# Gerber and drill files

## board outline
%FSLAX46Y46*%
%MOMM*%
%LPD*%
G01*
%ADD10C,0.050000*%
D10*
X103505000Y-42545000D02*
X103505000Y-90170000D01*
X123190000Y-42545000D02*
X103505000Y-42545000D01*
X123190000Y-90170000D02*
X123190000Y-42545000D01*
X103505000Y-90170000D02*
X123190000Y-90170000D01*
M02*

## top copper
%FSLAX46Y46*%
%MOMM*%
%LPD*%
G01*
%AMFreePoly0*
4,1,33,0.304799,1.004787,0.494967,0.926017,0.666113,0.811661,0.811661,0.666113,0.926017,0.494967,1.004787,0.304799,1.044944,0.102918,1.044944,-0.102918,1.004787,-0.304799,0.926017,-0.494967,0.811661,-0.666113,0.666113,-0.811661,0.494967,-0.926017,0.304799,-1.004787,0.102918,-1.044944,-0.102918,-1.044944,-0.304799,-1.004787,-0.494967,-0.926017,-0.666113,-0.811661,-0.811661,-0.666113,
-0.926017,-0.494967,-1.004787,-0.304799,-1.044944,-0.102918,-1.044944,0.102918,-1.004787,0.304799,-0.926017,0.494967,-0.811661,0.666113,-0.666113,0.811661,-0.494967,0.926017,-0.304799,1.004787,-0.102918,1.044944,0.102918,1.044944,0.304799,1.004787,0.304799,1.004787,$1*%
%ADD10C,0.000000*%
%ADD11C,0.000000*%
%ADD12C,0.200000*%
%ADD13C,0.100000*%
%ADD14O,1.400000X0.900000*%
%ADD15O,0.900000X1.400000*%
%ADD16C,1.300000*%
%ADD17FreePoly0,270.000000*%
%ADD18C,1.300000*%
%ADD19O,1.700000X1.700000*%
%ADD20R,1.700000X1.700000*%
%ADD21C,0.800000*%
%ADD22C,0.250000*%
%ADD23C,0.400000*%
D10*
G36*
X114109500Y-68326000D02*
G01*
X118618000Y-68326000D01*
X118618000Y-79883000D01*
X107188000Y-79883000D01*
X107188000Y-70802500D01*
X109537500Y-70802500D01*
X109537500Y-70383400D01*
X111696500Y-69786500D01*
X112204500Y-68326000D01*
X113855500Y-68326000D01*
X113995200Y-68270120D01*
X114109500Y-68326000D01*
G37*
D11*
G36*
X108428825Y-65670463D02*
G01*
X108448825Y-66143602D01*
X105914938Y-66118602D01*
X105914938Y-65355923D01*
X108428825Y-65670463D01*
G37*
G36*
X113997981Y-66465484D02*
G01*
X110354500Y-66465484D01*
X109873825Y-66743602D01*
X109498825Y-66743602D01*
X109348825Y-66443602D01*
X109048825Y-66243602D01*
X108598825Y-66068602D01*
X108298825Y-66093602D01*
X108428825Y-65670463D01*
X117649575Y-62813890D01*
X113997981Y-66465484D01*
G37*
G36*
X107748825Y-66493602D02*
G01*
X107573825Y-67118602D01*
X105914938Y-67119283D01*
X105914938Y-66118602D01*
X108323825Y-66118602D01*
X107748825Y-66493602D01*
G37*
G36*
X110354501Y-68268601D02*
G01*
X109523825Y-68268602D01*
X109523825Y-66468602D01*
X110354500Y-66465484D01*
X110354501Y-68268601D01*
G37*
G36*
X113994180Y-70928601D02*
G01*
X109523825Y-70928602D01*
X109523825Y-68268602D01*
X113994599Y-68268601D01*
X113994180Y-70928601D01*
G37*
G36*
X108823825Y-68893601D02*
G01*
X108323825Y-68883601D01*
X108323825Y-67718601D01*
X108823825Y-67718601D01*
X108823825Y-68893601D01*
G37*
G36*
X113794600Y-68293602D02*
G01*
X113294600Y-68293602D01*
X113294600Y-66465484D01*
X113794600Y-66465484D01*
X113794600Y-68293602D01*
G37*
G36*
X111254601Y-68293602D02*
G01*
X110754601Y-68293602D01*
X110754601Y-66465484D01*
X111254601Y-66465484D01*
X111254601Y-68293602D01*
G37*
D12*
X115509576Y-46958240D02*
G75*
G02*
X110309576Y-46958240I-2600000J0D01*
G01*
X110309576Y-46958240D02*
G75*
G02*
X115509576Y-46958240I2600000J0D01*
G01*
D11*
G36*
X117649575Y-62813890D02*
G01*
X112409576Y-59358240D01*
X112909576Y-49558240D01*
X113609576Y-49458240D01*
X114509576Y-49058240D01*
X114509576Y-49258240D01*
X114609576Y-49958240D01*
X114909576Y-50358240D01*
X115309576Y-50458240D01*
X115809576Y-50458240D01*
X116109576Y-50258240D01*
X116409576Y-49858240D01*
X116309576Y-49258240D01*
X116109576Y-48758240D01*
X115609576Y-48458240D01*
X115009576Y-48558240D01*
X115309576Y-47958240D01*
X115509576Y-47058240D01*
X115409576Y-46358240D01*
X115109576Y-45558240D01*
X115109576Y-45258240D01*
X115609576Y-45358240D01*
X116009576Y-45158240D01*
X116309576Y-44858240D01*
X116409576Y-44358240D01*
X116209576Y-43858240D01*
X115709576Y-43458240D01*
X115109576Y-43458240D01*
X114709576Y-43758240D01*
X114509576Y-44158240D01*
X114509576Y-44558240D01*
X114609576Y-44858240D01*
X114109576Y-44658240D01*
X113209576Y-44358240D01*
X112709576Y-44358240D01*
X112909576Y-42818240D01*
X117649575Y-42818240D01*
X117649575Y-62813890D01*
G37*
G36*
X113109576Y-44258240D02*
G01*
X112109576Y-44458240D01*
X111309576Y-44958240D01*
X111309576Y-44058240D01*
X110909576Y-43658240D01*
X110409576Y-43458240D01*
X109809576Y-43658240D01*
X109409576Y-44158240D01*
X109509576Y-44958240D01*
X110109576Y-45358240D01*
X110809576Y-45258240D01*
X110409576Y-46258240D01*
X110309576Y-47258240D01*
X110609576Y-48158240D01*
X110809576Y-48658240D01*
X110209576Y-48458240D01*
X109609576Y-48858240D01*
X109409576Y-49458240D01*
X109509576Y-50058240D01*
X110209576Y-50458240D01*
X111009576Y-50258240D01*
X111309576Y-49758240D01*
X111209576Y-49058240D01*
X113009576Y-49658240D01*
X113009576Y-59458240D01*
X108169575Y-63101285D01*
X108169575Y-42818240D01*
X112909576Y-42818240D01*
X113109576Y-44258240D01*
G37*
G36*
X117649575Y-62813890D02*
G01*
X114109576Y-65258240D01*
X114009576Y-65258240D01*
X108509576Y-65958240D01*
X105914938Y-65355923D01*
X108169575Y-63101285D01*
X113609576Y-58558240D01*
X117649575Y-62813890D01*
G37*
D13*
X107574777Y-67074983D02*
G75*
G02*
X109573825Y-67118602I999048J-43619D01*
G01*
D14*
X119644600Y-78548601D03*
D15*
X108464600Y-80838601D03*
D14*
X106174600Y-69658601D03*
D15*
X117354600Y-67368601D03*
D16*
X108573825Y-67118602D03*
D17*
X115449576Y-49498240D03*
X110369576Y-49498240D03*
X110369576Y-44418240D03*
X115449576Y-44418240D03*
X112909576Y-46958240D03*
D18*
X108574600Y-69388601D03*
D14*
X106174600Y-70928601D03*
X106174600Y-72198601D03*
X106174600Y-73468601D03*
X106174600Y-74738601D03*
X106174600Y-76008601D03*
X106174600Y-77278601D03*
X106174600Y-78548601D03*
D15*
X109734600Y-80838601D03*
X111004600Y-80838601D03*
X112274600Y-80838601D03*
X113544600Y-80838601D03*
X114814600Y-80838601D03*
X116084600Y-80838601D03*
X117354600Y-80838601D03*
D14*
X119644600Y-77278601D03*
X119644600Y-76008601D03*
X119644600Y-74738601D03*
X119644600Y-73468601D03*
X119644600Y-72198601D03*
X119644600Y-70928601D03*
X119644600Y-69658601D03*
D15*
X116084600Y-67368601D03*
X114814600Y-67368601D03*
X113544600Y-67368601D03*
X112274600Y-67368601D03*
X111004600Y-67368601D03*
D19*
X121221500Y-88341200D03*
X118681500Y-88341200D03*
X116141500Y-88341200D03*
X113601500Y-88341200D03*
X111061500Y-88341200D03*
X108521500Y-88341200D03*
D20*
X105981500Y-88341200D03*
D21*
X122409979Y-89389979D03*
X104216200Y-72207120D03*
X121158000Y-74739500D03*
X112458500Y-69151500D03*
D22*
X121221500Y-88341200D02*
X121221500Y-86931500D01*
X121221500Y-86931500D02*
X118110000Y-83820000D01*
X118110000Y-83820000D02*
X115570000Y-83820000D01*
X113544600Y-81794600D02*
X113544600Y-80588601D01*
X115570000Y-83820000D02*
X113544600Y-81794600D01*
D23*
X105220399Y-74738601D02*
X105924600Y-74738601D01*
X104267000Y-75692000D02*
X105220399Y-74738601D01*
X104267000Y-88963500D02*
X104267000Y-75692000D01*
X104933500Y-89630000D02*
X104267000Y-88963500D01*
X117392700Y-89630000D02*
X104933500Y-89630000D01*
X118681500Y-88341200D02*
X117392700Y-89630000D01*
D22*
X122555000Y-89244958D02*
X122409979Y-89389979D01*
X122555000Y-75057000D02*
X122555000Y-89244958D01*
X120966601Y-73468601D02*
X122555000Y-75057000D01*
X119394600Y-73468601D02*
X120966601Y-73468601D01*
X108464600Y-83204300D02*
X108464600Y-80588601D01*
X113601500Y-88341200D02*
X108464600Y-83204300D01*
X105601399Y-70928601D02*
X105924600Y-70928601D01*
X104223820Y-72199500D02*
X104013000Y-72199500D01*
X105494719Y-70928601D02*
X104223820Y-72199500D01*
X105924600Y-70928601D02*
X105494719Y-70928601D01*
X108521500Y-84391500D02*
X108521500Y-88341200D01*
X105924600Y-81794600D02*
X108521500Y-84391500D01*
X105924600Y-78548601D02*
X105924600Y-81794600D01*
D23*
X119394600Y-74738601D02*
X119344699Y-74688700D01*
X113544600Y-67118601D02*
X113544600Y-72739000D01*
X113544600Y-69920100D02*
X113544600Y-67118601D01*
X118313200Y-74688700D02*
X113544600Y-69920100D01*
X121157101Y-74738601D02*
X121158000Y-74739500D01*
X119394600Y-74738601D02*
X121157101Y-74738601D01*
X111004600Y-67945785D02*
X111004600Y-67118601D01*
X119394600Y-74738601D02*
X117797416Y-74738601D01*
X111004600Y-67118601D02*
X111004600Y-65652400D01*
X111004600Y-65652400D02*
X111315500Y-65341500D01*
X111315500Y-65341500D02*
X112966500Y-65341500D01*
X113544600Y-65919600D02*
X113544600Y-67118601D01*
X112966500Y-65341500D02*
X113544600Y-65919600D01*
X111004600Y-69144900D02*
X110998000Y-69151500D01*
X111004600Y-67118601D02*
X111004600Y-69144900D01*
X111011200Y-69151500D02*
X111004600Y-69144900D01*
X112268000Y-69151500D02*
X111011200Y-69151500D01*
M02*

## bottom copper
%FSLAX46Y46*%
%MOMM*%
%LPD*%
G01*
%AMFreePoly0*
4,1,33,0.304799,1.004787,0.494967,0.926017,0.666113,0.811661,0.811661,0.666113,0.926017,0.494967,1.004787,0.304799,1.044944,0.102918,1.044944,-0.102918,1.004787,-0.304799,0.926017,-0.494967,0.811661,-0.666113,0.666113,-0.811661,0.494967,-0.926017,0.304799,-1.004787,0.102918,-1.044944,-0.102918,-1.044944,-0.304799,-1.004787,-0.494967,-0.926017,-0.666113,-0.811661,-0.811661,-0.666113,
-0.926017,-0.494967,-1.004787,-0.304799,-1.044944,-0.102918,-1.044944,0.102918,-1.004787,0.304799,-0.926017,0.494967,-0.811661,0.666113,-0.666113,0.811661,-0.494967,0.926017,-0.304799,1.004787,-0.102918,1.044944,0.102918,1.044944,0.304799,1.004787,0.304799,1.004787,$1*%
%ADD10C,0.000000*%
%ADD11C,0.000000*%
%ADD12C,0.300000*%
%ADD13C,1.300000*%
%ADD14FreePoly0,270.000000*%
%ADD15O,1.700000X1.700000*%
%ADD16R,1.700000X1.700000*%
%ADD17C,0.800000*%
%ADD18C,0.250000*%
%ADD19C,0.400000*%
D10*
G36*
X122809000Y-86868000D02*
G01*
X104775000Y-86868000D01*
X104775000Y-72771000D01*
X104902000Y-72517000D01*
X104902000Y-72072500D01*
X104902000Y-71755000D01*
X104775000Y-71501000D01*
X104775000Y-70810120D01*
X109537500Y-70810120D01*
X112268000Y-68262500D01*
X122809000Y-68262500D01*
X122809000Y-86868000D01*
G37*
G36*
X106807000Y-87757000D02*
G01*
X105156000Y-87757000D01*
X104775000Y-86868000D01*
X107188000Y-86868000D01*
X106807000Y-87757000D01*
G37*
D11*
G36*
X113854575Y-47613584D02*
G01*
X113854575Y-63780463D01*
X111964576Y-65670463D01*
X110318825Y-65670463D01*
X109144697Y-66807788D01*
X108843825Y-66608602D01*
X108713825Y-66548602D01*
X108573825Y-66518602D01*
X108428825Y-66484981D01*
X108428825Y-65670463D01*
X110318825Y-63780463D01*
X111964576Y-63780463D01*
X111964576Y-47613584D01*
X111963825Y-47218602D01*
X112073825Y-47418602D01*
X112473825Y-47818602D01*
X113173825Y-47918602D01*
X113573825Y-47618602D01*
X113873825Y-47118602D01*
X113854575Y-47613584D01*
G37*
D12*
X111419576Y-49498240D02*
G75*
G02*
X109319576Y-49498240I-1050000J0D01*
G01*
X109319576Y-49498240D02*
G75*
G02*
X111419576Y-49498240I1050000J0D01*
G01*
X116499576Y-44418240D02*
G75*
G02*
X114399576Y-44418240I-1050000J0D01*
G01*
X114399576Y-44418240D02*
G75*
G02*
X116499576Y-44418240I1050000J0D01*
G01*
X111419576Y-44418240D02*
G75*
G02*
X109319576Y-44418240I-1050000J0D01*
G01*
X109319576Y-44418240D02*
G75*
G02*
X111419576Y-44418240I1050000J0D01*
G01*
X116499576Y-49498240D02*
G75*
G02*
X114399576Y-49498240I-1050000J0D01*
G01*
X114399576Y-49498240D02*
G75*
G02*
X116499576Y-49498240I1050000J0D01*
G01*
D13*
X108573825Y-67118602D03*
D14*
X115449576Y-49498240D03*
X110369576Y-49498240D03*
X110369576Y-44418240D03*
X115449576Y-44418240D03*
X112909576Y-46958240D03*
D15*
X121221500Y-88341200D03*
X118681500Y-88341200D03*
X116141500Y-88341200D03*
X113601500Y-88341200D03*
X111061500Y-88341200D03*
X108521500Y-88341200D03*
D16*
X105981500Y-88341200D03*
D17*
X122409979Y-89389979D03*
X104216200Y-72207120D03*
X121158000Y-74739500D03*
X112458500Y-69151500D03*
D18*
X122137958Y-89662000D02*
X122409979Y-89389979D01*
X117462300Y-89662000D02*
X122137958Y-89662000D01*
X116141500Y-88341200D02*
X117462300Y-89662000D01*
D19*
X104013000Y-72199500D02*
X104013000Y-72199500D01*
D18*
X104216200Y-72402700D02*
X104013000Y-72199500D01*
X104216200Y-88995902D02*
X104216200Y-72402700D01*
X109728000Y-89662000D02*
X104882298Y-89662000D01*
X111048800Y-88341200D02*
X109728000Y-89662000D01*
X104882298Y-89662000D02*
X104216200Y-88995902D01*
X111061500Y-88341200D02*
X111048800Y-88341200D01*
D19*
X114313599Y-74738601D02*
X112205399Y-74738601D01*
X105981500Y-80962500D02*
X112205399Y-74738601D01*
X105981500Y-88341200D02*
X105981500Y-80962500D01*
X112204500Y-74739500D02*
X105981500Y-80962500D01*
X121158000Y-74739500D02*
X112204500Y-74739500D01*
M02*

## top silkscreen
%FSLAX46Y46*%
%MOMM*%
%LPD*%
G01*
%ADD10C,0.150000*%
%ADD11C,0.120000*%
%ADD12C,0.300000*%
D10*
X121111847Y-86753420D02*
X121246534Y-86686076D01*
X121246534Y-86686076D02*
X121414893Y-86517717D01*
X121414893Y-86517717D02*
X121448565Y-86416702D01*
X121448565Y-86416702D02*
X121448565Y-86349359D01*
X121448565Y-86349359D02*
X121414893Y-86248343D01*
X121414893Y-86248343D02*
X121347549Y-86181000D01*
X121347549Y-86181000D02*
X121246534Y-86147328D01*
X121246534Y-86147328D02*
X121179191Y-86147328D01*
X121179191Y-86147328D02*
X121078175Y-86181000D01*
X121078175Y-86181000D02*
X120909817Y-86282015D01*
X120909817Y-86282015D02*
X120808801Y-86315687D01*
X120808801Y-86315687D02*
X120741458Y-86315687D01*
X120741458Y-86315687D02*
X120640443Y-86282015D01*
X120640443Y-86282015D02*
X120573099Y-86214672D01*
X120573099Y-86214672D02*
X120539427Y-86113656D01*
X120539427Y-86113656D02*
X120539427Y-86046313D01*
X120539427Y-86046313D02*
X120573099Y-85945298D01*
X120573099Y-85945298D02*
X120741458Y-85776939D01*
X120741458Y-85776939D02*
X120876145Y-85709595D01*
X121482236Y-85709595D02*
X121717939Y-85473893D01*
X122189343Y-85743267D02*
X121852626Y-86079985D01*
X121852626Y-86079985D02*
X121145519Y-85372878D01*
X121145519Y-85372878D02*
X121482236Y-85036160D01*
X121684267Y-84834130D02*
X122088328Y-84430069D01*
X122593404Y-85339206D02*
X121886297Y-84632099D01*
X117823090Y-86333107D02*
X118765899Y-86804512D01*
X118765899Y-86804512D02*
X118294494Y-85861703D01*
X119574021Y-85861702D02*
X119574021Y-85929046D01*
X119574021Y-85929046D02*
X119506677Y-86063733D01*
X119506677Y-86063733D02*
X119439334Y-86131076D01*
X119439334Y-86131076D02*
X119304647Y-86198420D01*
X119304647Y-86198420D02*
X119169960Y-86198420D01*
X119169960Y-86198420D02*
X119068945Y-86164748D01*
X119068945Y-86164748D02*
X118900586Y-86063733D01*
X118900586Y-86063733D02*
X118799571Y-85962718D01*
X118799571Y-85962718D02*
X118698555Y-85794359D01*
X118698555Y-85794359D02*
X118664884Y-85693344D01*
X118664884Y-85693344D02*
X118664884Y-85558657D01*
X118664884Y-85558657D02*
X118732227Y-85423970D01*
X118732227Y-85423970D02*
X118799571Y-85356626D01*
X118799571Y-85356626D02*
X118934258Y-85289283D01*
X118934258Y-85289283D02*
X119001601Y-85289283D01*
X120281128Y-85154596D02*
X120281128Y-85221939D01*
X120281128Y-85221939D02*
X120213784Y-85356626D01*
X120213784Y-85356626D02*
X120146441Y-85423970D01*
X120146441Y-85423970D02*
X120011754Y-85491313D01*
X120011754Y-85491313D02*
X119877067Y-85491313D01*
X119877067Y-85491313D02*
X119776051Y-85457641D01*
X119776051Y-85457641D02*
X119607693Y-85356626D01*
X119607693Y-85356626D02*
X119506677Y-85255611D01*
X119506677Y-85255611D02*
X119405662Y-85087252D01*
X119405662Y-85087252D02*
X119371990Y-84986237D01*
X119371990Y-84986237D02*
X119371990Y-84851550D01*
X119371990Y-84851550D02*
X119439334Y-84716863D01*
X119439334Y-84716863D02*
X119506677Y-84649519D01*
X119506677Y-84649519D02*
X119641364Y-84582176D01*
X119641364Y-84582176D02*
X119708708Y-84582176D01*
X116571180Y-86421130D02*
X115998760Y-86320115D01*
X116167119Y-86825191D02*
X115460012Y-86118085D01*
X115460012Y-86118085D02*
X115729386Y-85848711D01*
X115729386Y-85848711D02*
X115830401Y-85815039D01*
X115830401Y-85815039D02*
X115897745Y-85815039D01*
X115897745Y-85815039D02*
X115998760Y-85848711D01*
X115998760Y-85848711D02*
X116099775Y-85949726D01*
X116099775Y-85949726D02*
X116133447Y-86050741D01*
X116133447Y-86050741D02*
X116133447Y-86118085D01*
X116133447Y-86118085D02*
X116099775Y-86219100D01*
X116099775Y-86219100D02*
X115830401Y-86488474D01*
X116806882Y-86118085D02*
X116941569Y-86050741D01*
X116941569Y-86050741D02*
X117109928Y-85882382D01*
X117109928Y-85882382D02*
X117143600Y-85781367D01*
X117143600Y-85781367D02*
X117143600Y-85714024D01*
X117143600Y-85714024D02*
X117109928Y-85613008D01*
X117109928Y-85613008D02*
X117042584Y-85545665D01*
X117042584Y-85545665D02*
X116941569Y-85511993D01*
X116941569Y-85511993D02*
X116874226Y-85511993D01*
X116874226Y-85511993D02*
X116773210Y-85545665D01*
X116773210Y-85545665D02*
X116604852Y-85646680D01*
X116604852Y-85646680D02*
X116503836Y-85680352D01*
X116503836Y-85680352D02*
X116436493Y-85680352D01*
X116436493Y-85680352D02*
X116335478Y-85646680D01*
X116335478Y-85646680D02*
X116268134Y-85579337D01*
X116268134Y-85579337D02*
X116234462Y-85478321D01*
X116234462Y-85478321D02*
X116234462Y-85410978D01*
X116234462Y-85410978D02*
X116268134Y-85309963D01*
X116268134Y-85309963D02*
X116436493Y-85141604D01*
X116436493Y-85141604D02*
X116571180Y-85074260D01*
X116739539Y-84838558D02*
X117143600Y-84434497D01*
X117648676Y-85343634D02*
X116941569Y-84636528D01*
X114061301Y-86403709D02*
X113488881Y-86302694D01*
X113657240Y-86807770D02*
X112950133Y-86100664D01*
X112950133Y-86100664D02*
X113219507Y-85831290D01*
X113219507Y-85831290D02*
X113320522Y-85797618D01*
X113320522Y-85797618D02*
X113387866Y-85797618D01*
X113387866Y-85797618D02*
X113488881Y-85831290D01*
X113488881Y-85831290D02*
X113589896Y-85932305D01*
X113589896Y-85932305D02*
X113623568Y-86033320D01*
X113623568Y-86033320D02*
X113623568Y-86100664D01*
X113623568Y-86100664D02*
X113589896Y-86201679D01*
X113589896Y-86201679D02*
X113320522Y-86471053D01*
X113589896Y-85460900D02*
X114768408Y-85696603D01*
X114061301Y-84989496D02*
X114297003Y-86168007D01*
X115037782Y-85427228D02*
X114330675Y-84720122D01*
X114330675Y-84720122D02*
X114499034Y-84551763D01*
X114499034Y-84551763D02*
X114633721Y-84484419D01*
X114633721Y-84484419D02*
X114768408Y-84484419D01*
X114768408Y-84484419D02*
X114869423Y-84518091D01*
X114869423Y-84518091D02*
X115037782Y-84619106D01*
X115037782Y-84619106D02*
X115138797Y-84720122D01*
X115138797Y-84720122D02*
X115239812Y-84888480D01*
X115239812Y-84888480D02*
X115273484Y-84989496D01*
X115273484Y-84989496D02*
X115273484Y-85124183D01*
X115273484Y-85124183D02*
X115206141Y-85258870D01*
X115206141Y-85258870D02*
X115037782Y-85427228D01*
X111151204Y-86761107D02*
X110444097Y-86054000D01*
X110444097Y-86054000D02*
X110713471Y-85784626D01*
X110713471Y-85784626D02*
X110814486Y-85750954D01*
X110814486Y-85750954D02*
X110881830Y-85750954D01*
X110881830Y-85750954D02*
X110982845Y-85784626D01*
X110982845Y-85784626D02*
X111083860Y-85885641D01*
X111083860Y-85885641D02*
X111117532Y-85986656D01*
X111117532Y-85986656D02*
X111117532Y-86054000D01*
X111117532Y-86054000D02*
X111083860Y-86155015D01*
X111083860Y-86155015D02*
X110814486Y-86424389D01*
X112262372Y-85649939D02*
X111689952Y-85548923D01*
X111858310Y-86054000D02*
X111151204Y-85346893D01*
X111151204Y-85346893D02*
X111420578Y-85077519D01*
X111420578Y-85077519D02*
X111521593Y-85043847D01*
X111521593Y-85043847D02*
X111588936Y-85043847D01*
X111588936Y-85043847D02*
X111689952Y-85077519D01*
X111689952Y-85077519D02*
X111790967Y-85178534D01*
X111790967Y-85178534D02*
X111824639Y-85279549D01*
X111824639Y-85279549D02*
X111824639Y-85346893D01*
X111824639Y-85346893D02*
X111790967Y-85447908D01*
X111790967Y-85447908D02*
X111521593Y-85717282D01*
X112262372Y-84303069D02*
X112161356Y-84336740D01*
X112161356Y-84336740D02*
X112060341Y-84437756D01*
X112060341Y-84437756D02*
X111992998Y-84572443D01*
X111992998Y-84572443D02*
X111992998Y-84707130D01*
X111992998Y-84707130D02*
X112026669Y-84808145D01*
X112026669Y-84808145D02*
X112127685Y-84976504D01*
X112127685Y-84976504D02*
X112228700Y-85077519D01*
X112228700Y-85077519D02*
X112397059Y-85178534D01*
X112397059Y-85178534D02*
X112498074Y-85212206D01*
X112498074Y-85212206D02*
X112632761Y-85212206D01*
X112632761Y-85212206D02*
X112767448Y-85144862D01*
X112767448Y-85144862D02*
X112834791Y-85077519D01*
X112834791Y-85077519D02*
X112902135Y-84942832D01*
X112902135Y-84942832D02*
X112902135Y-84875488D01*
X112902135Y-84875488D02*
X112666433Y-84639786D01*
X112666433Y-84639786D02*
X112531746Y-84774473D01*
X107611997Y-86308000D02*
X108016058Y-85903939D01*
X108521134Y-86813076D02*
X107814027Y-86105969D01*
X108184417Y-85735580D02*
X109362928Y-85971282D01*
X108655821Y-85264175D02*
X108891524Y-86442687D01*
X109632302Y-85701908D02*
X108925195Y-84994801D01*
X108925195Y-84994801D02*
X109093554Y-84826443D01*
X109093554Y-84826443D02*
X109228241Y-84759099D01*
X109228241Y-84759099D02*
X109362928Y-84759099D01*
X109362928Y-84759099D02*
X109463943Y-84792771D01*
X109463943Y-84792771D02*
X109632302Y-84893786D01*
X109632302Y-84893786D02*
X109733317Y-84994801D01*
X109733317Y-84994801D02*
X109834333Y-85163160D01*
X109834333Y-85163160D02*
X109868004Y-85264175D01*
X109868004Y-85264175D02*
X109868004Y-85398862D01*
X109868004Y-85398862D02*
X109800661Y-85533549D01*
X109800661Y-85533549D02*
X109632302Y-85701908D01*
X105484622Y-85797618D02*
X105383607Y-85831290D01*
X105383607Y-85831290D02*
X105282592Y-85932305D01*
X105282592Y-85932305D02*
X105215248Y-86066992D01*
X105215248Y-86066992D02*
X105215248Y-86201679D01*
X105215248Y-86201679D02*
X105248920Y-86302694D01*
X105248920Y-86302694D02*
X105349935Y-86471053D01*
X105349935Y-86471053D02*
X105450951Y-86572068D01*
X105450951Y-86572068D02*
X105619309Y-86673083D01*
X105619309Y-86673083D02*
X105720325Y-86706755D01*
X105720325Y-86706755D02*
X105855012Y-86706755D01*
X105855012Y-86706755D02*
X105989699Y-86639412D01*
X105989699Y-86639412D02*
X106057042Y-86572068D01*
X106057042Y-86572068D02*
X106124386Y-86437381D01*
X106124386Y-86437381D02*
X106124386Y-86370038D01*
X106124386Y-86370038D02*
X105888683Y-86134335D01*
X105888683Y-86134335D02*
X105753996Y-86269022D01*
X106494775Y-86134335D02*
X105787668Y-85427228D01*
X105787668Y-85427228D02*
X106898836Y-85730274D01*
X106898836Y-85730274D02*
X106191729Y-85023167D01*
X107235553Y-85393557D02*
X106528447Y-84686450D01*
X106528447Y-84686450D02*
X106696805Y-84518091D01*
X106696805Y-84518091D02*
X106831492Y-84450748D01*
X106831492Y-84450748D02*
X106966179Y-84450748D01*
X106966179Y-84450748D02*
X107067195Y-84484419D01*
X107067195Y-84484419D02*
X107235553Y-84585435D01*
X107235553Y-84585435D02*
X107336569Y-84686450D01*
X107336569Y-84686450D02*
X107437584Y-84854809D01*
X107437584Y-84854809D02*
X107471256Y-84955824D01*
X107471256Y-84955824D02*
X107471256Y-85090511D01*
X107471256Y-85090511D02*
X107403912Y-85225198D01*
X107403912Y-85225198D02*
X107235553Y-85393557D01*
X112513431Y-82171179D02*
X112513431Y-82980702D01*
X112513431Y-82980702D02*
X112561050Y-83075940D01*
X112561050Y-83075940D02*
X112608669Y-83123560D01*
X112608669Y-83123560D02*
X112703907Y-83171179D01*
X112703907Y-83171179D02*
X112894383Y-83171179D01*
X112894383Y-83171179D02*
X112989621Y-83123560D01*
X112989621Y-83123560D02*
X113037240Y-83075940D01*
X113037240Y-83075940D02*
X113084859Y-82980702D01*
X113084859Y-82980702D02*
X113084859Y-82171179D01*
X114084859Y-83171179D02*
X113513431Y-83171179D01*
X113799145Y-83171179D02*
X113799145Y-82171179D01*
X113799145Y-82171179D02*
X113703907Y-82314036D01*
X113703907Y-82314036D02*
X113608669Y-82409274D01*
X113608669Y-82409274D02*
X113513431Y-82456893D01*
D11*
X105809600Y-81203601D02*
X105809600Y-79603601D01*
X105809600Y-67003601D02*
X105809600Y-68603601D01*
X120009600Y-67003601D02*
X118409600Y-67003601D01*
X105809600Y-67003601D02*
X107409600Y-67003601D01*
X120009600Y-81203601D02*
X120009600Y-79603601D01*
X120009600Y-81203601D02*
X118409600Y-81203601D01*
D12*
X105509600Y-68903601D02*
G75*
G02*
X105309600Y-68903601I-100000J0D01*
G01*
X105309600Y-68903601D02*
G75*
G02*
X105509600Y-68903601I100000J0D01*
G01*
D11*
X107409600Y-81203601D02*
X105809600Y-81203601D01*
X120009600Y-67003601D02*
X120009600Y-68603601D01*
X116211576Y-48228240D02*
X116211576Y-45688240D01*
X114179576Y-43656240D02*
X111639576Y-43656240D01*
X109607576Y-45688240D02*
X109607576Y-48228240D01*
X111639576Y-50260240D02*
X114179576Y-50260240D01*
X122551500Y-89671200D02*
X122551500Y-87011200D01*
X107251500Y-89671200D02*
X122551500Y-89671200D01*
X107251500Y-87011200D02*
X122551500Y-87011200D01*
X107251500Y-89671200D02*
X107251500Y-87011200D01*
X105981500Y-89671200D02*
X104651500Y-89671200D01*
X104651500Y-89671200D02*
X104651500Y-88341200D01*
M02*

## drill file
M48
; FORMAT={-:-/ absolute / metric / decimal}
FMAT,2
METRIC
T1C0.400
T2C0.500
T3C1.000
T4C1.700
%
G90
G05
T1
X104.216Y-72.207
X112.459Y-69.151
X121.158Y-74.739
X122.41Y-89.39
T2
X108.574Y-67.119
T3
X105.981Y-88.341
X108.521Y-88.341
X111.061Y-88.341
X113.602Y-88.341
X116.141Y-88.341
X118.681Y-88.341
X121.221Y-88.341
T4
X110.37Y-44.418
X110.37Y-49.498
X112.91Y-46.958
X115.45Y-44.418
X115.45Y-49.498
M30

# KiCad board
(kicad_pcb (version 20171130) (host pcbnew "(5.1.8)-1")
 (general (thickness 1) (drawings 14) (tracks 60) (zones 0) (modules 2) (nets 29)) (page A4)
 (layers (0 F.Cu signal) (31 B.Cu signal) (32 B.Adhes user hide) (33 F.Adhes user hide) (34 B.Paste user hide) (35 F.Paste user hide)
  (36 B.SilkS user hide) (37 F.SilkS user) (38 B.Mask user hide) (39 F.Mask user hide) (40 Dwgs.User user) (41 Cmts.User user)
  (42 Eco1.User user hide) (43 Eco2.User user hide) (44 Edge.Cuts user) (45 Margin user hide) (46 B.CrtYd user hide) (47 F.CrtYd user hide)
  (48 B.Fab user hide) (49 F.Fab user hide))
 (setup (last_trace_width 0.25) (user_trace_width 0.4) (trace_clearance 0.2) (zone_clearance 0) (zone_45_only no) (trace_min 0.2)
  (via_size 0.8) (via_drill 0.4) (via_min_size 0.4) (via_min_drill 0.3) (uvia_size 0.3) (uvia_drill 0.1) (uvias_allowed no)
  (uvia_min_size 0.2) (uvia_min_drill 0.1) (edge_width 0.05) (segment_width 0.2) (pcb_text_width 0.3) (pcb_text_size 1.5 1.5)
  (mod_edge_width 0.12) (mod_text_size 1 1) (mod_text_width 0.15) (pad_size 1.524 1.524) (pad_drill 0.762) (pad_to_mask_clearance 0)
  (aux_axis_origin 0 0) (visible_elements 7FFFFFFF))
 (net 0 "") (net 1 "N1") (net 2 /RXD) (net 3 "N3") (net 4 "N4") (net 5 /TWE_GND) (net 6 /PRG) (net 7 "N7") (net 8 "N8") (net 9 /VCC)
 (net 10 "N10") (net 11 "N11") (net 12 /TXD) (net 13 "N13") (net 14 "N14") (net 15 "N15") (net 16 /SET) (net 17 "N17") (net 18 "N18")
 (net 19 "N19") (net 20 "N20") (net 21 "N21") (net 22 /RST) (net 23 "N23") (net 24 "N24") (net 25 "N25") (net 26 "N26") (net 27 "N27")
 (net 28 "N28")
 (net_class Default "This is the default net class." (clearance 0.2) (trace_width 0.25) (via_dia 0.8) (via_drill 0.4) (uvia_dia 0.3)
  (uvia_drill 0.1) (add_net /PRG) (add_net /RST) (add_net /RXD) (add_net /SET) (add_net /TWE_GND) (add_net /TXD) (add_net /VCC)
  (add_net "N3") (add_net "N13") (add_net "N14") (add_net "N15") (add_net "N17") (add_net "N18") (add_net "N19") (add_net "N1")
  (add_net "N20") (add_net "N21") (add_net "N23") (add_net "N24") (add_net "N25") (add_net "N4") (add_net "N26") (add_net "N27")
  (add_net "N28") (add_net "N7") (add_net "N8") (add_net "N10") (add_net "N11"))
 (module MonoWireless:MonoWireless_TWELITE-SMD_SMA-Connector (layer F.Cu) (at 112.9096 74.103601)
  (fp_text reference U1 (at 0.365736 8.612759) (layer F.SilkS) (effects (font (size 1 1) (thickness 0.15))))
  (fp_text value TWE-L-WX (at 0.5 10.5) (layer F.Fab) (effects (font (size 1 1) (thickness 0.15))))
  (fp_line (start -7.1 7.1) (end -7.1 5.5) (layer F.SilkS) (width 0.12))
  (fp_line (start -7.1 -7.1) (end -7.1 -5.5) (layer F.SilkS) (width 0.12))
  (fp_line (start 7.1 -7.1) (end 5.5 -7.1) (layer F.SilkS) (width 0.12))
  (fp_line (start -7.1 -7.1) (end -5.5 -7.1) (layer F.SilkS) (width 0.12))
  (fp_line (start 7.1 7.1) (end 7.1 5.5) (layer F.SilkS) (width 0.12))
  (fp_line (start 7.1 7.1) (end 5.5 7.1) (layer F.SilkS) (width 0.12))
  (fp_circle (center -7.5 -5.2) (end -7.4 -5.2) (layer F.SilkS) (width 0.3))
  (fp_line (start -5.5 7.1) (end -7.1 7.1) (layer F.SilkS) (width 0.12))
  (fp_line (start 7.1 -7.1) (end 7.1 -5.5) (layer F.SilkS) (width 0.12))
  (fp_poly (pts (xy -4.480775 -8.433138) (xy -4.460775 -7.959999) (xy -6.994662 -7.984999) (xy -6.994662 -8.747678)) (layer F.Cu) (width 0))
  (fp_poly
   (pts (xy -4.610775 -8.009999) (xy -4.480775 -8.433138) (xy 4.739975 -11.289711) (xy 1.088381 -7.638117) (xy -2.5551 -7.638117)
    (xy -3.035775 -7.359999) (xy -3.410775 -7.359999) (xy -3.560775 -7.659999) (xy -3.860775 -7.859999) (xy -4.310775 -8.034999))
   (layer F.Cu) (width 0))
  (fp_poly
   (pts (xy -5.160775 -7.609999) (xy -5.335775 -6.984999) (xy -6.994662 -6.984318) (xy -6.994662 -7.984999) (xy -4.585775 -7.984999))
   (layer F.Cu) (width 0))
  (fp_poly
   (pts (xy -2.5551 -7.638117) (xy -2.555099 -5.835) (xy -3.385775 -5.834999) (xy -3.385775 -7.634999) (xy -2.5551 -7.638117)) (layer F.Cu)
   (width 0))
  (fp_poly (pts (xy 1.08458 -3.175) (xy -3.385775 -3.174999) (xy -3.385775 -5.834999) (xy 1.084999 -5.835)) (layer F.Cu) (width 0))
  (fp_poly (pts (xy -4.085775 -5.21) (xy -4.585775 -5.22) (xy -4.585775 -6.385) (xy -4.085775 -6.385)) (layer F.Cu) (width 0))
  (fp_poly (pts (xy 0.885 -5.809999) (xy 0.385 -5.809999) (xy 0.385 -7.638117) (xy 0.885 -7.638117)) (layer F.Cu) (width 0))
  (fp_poly (pts (xy -1.654999 -5.809999) (xy -2.154999 -5.809999) (xy -2.154999 -7.638117) (xy -1.654999 -7.638117)) (layer F.Cu) (width 0))
  (fp_circle (center -0.000024 -27.145361) (end 2.599976 -27.145361) (layer F.Cu) (width 0.2))
  (fp_poly
   (pts (xy 4.739975 -11.289711) (xy -0.500024 -14.745361) (xy -0.000024 -24.545361) (xy 0.699976 -24.645361) (xy 1.599976 -25.045361)
    (xy 1.599976 -24.845361) (xy 1.699976 -24.145361) (xy 1.999976 -23.745361) (xy 2.399976 -23.645361) (xy 2.899976 -23.645361)
    (xy 3.199976 -23.845361) (xy 3.499976 -24.245361) (xy 3.399976 -24.845361) (xy 3.199976 -25.345361) (xy 2.699976 -25.645361)
    (xy 2.099976 -25.545361) (xy 2.399976 -26.145361) (xy 2.599976 -27.045361) (xy 2.499976 -27.745361) (xy 2.199976 -28.545361)
    (xy 2.199976 -28.845361) (xy 2.699976 -28.745361) (xy 3.099976 -28.945361) (xy 3.399976 -29.245361) (xy 3.499976 -29.745361)
    (xy 3.299976 -30.245361) (xy 2.799976 -30.645361) (xy 2.199976 -30.645361) (xy 1.799976 -30.345361) (xy 1.599976 -29.945361)
    (xy 1.599976 -29.545361) (xy 1.699976 -29.245361) (xy 1.199976 -29.445361) (xy 0.299976 -29.745361) (xy -0.200024 -29.745361)
    (xy -0.000024 -31.285361) (xy 4.739975 -31.285361))
   (layer F.Cu) (width 0))
  (fp_poly
   (pts (xy 0.199976 -29.845361) (xy -0.800024 -29.645361) (xy -1.600024 -29.145361) (xy -1.600024 -30.045361) (xy -2.000024 -30.445361)
    (xy -2.500024 -30.645361) (xy -3.100024 -30.445361) (xy -3.500024 -29.945361) (xy -3.400024 -29.145361) (xy -2.800024 -28.745361)
    (xy -2.100024 -28.845361) (xy -2.500024 -27.845361) (xy -2.600024 -26.845361) (xy -2.300024 -25.945361) (xy -2.100024 -25.445361)
    (xy -2.700024 -25.645361) (xy -3.300024 -25.245361) (xy -3.500024 -24.645361) (xy -3.400024 -24.045361) (xy -2.700024 -23.645361)
    (xy -1.900024 -23.845361) (xy -1.600024 -24.345361) (xy -1.700024 -25.045361) (xy 0.099976 -24.445361) (xy 0.099976 -14.645361)
    (xy -4.740025 -11.002316) (xy -4.740025 -31.285361) (xy -0.000024 -31.285361))
   (layer F.Cu) (width 0))
  (fp_poly
   (pts (xy 4.739975 -11.289711) (xy 1.199976 -8.845361) (xy 1.099976 -8.845361) (xy -4.400024 -8.145361) (xy -6.994662 -8.747678)
    (xy -4.740025 -11.002316) (xy 0.699976 -15.545361))
   (layer F.Cu) (width 0))
  (fp_poly
   (pts (xy -0.835775 -26.684999) (xy -0.435775 -26.284999) (xy 0.264225 -26.184999) (xy 0.664225 -26.484999) (xy 0.964225 -26.984999)
    (xy 0.944975 -26.490017) (xy 0.944975 -10.323138) (xy -0.945024 -8.433138) (xy -2.590775 -8.433138) (xy -3.764903 -7.295813)
    (xy -4.065775 -7.494999) (xy -4.195775 -7.554999) (xy -4.335775 -7.584999) (xy -4.480775 -7.61862) (xy -4.480775 -8.433138)
    (xy -2.590775 -10.323138) (xy -0.945024 -10.323138) (xy -0.945024 -26.490017) (xy -0.945775 -26.884999))
   (layer B.Cu) (width 0))
  (fp_circle (center -2.540024 -24.605361) (end -1.490024 -24.605361) (layer B.Cu) (width 0.3))
  (fp_circle (center 2.539976 -29.685361) (end 3.589976 -29.685361) (layer B.Cu) (width 0.3))
  (fp_circle (center -2.540024 -29.685361) (end -1.490024 -29.685361) (layer B.Cu) (width 0.3))
  (fp_circle (center 2.539976 -24.605361) (end 3.589976 -24.605361) (layer B.Cu) (width 0.3))
  (fp_line (start 3.301976 -25.875361) (end 3.301976 -28.415361) (layer F.SilkS) (width 0.12))
  (fp_line (start 1.269976 -30.447361) (end -1.270024 -30.447361) (layer F.SilkS) (width 0.12))
  (fp_line (start -3.302024 -28.415361) (end -3.302024 -25.875361) (layer F.SilkS) (width 0.12))
  (fp_line (start -1.270024 -23.843361) (end 1.269976 -23.843361) (layer F.SilkS) (width 0.12))
  (fp_arc (start -4.335775 -6.984999) (end -3.335775 -6.984999) (angle -177.5) (layer F.Cu) (width 0.1))
  (pad 17 smd oval (at 6.735 4.445) (size 1.4 0.9) (layers F.Cu F.Paste F.Mask) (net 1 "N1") (zone_connect 0))
  (pad 9 smd oval (at -4.445 6.735 270) (size 1.4 0.9) (layers F.Cu F.Paste F.Mask) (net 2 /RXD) (zone_connect 0))
  (pad 1 smd oval (at -6.735 -4.445 180) (size 1.4 0.9) (layers F.Cu F.Paste F.Mask) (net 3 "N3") (zone_connect 0))
  (pad 25 smd oval (at 4.445 -6.735 90) (size 1.4 0.9) (layers F.Cu F.Paste F.Mask) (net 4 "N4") (zone_connect 0))
  (pad "" thru_hole circle (at -4.335775 -6.984999) (size 1.3 1.3) (drill 0.5) (layers *.Cu B.Mask) (zone_connect 0))
  (pad "" thru_hole custom (at 2.539976 -24.605361 270) (size 2.1 2.1) (drill 1.7) (layers *.Cu *.Mask) (zone_connect 0)
   (options (clearance outline) (anchor circle)) (primitives))
  (pad "" thru_hole custom (at -2.540024 -24.605361 270) (size 2.1 2.1) (drill 1.7) (layers *.Cu *.Mask) (zone_connect 0)
   (options (clearance outline) (anchor circle)) (primitives))
  (pad "" thru_hole custom (at -2.540024 -29.685361 270) (size 2.1 2.1) (drill 1.7) (layers *.Cu *.Mask) (zone_connect 0)
   (options (clearance outline) (anchor circle)) (primitives))
  (pad "" thru_hole custom (at 2.539976 -29.685361 270) (size 2.1 2.1) (drill 1.7) (layers *.Cu *.Mask) (zone_connect 0)
   (options (clearance outline) (anchor circle)) (primitives))
  (pad "" thru_hole custom (at -0.000024 -27.145361 270) (size 2.1 2.1) (drill 1.7) (layers *.Cu *.Mask) (zone_connect 0)
   (options (clearance outline) (anchor circle)) (primitives))
  (pad "" smd circle (at -4.335 -4.715) (size 1.3 1.3) (layers F.Cu F.Mask) (zone_connect 0))
  (pad 31 smd custom (at -6.6 -11.9 270) (size 0.9 0.9) (layers Dwgs.User) (zone_connect 0) (options (clearance outline) (anchor circle))
   (primitives))
  (pad 32 smd custom (at -5.5 -11.9 270) (size 0.9 0.9) (layers Dwgs.User) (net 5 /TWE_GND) (zone_connect 0)
   (options (clearance outline) (anchor circle)) (primitives))
  (pad 2 smd oval (at -6.735 -3.175 180) (size 1.4 0.9) (layers F.Cu F.Paste F.Mask) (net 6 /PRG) (zone_connect 0))
  (pad 3 smd oval (at -6.735 -1.905 180) (size 1.4 0.9) (layers F.Cu F.Paste F.Mask) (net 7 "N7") (zone_connect 0))
  (pad 4 smd oval (at -6.735 -0.635 180) (size 1.4 0.9) (layers F.Cu F.Paste F.Mask) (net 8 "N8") (zone_connect 0))
  (pad 5 smd oval (at -6.735 0.635 180) (size 1.4 0.9) (layers F.Cu F.Paste F.Mask) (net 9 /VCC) (zone_connect 0))
  (pad 6 smd oval (at -6.735 1.905 180) (size 1.4 0.9) (layers F.Cu F.Paste F.Mask) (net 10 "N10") (zone_connect 0))
  (pad 7 smd oval (at -6.735 3.175 180) (size 1.4 0.9) (layers F.Cu F.Paste F.Mask) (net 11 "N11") (zone_connect 0))
  (pad 8 smd oval (at -6.735 4.445 180) (size 1.4 0.9) (layers F.Cu F.Paste F.Mask) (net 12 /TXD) (zone_connect 0))
  (pad 10 smd oval (at -3.175 6.735 270) (size 1.4 0.9) (layers F.Cu F.Paste F.Mask) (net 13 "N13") (zone_connect 0))
  (pad 11 smd oval (at -1.905 6.735 270) (size 1.4 0.9) (layers F.Cu F.Paste F.Mask) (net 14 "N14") (zone_connect 0))
  (pad 12 smd oval (at -0.635 6.735 270) (size 1.4 0.9) (layers F.Cu F.Paste F.Mask) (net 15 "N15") (zone_connect 0))
  (pad 13 smd oval (at 0.635 6.735 270) (size 1.4 0.9) (layers F.Cu F.Paste F.Mask) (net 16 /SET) (zone_connect 0))
  (pad 14 smd oval (at 1.905 6.735 270) (size 1.4 0.9) (layers F.Cu F.Paste F.Mask) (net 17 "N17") (zone_connect 0))
  (pad 15 smd oval (at 3.175 6.735 270) (size 1.4 0.9) (layers F.Cu F.Paste F.Mask) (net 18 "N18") (zone_connect 0))
  (pad 16 smd oval (at 4.445 6.735 270) (size 1.4 0.9) (layers F.Cu F.Paste F.Mask) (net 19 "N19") (zone_connect 0))
  (pad 18 smd oval (at 6.735 3.175) (size 1.4 0.9) (layers F.Cu F.Paste F.Mask) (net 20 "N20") (zone_connect 0))
  (pad 19 smd oval (at 6.735 1.905) (size 1.4 0.9) (layers F.Cu F.Paste F.Mask) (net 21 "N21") (zone_connect 0))
  (pad 20 smd oval (at 6.735 0.635) (size 1.4 0.9) (layers F.Cu F.Paste F.Mask) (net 5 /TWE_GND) (zone_connect 0))
  (pad 21 smd oval (at 6.735 -0.635) (size 1.4 0.9) (layers F.Cu F.Paste F.Mask) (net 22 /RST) (zone_connect 0))
  (pad 22 smd oval (at 6.735 -1.905) (size 1.4 0.9) (layers F.Cu F.Paste F.Mask) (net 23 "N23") (zone_connect 0))
  (pad 23 smd oval (at 6.735 -3.175) (size 1.4 0.9) (layers F.Cu F.Paste F.Mask) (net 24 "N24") (zone_connect 0))
  (pad 24 smd oval (at 6.735 -4.445) (size 1.4 0.9) (layers F.Cu F.Paste F.Mask) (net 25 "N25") (zone_connect 0))
  (pad 26 smd oval (at 3.175 -6.735 90) (size 1.4 0.9) (layers F.Cu F.Paste F.Mask) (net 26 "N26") (zone_connect 0))
  (pad 27 smd oval (at 1.905 -6.735 90) (size 1.4 0.9) (layers F.Cu F.Paste F.Mask) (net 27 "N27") (zone_connect 0))
  (pad 28 smd oval (at 0.635 -6.735 90) (size 1.4 0.9) (layers F.Cu F.Paste F.Mask) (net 5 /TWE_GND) (zone_connect 0))
  (pad 29 smd oval (at -0.635 -6.735 90) (size 1.4 0.9) (layers F.Cu F.Paste F.Mask) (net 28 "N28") (zone_connect 0))
  (pad 30 smd oval (at -1.905 -6.735 90) (size 1.4 0.9) (layers F.Cu F.Paste F.Mask) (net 5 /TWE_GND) (zone_connect 0)))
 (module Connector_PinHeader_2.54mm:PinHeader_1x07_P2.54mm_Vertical (layer F.Cu) (at 105.9815 88.3412 90)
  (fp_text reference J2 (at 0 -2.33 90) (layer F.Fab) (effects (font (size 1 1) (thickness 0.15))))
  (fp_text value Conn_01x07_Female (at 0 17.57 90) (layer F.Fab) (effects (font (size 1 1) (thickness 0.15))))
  (fp_line (start -1.33 16.57) (end 1.33 16.57) (layer F.SilkS) (width 0.12))
  (fp_line (start -1.33 1.27) (end -1.33 16.57) (layer F.SilkS) (width 0.12))
  (fp_line (start 1.33 1.27) (end 1.33 16.57) (layer F.SilkS) (width 0.12))
  (fp_line (start -1.33 1.27) (end 1.33 1.27) (layer F.SilkS) (width 0.12))
  (fp_line (start -1.33 0) (end -1.33 -1.33) (layer F.SilkS) (width 0.12))
  (fp_line (start -1.33 -1.33) (end 0 -1.33) (layer F.SilkS) (width 0.12))
  (pad 7 thru_hole oval (at 0 15.24 90) (size 1.7 1.7) (drill 1) (layers *.Cu *.Mask) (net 16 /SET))
  (pad 6 thru_hole oval (at 0 12.7 90) (size 1.7 1.7) (drill 1) (layers *.Cu *.Mask) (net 9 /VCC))
  (pad 5 thru_hole oval (at 0 10.16 90) (size 1.7 1.7) (drill 1) (layers *.Cu *.Mask) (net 22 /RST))
  (pad 4 thru_hole oval (at 0 7.62 90) (size 1.7 1.7) (drill 1) (layers *.Cu *.Mask) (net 2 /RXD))
  (pad 3 thru_hole oval (at 0 5.08 90) (size 1.7 1.7) (drill 1) (layers *.Cu *.Mask) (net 6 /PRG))
  (pad 2 thru_hole oval (at 0 2.54 90) (size 1.7 1.7) (drill 1) (layers *.Cu *.Mask) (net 12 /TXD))
  (pad 1 thru_hole rect (at 0 0 90) (size 1.7 1.7) (drill 1) (layers *.Cu *.Mask) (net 5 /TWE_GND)))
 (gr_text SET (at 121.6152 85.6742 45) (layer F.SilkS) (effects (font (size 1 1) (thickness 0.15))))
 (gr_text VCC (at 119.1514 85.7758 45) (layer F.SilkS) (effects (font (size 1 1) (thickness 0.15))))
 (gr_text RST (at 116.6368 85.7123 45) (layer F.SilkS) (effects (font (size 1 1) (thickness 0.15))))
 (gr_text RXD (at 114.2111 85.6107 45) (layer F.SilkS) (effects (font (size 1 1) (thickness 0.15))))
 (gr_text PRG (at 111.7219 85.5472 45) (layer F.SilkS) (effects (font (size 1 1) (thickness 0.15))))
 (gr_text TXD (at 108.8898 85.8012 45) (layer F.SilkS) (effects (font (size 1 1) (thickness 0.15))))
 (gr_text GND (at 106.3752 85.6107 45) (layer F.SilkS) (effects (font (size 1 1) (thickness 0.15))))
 (gr_poly
  (pts (xy 122.809 86.868) (xy 104.775 86.868) (xy 104.775 72.771) (xy 104.902 72.517) (xy 104.902 72.0725) (xy 104.902 71.755)
   (xy 104.775 71.501) (xy 104.775 70.81012) (xy 109.5375 70.81012) (xy 112.268 68.2625) (xy 122.809 68.2625))
  (layer B.Cu) (width 0))
 (gr_poly (pts (xy 106.807 87.757) (xy 105.156 87.757) (xy 104.775 86.868) (xy 107.188 86.868)) (layer B.Cu) (width 0))
 (gr_poly
  (pts (xy 113.8555 68.326) (xy 113.9952 68.27012) (xy 114.1095 68.326) (xy 118.618 68.326) (xy 118.618 79.883) (xy 107.188 79.883)
   (xy 107.188 70.8025) (xy 109.5375 70.8025) (xy 109.5375 70.3834) (xy 111.6965 69.7865) (xy 112.2045 68.326))
  (layer F.Cu) (width 0))
 (gr_line (start 103.505 42.545) (end 103.505 90.17) (layer Edge.Cuts) (width 0.05))
 (gr_line (start 123.19 42.545) (end 103.505 42.545) (layer Edge.Cuts) (width 0.05))
 (gr_line (start 123.19 90.17) (end 123.19 42.545) (layer Edge.Cuts) (width 0.05))
 (gr_line (start 103.505 90.17) (end 123.19 90.17) (layer Edge.Cuts) (width 0.05))
 (segment (start 121.2215 88.3412) (end 121.2215 86.9315) (width 0.25) (layer F.Cu) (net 16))
 (segment (start 121.2215 86.9315) (end 118.11 83.82) (width 0.25) (layer F.Cu) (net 16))
 (segment (start 118.11 83.82) (end 115.57 83.82) (width 0.25) (layer F.Cu) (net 16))
 (segment (start 113.5446 81.7946) (end 113.5446 80.588601) (width 0.25) (layer F.Cu) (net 16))
 (segment (start 115.57 83.82) (end 113.5446 81.7946) (width 0.25) (layer F.Cu) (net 16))
 (segment (start 105.220399 74.738601) (end 105.9246 74.738601) (width 0.4) (layer F.Cu) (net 9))
 (segment (start 104.267 75.692) (end 105.220399 74.738601) (width 0.4) (layer F.Cu) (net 9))
 (segment (start 104.267 88.9635) (end 104.267 75.692) (width 0.4) (layer F.Cu) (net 9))
 (segment (start 104.9335 89.63) (end 104.267 88.9635) (width 0.4) (layer F.Cu) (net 9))
 (segment (start 117.3927 89.63) (end 104.9335 89.63) (width 0.4) (layer F.Cu) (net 9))
 (segment (start 118.6815 88.3412) (end 117.3927 89.63) (width 0.4) (layer F.Cu) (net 9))
 (via (at 122.409979 89.389979) (size 0.8) (drill 0.4) (layers F.Cu B.Cu) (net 22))
 (segment (start 122.137958 89.662) (end 122.409979 89.389979) (width 0.25) (layer B.Cu) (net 22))
 (segment (start 117.4623 89.662) (end 122.137958 89.662) (width 0.25) (layer B.Cu) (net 22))
 (segment (start 116.1415 88.3412) (end 117.4623 89.662) (width 0.25) (layer B.Cu) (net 22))
 (segment (start 122.555 89.244958) (end 122.409979 89.389979) (width 0.25) (layer F.Cu) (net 22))
 (segment (start 122.555 75.057) (end 122.555 89.244958) (width 0.25) (layer F.Cu) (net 22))
 (segment (start 120.966601 73.468601) (end 122.555 75.057) (width 0.25) (layer F.Cu) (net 22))
 (segment (start 119.3946 73.468601) (end 120.966601 73.468601) (width 0.25) (layer F.Cu) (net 22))
 (segment (start 108.4646 83.2043) (end 108.4646 80.588601) (width 0.25) (layer F.Cu) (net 2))
 (segment (start 113.6015 88.3412) (end 108.4646 83.2043) (width 0.25) (layer F.Cu) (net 2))
 (segment (start 105.601399 70.928601) (end 105.9246 70.928601) (width 0.25) (layer F.Cu) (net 6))
 (segment (start 104.013 72.1995) (end 104.013 72.1995) (width 0.4) (layer B.Cu) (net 6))
 (via (at 104.2162 72.20712) (size 0.8) (drill 0.4) (layers F.Cu B.Cu) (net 6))
 (segment (start 104.22382 72.1995) (end 104.013 72.1995) (width 0.25) (layer F.Cu) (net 6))
 (segment (start 105.494719 70.928601) (end 104.22382 72.1995) (width 0.25) (layer F.Cu) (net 6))
 (segment (start 105.9246 70.928601) (end 105.494719 70.928601) (width 0.25) (layer F.Cu) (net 6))
 (segment (start 104.2162 72.4027) (end 104.013 72.1995) (width 0.25) (layer B.Cu) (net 6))
 (segment (start 104.2162 88.995902) (end 104.2162 72.4027) (width 0.25) (layer B.Cu) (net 6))
 (segment (start 109.728 89.662) (end 104.882298 89.662) (width 0.25) (layer B.Cu) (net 6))
 (segment (start 111.0488 88.3412) (end 109.728 89.662) (width 0.25) (layer B.Cu) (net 6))
 (segment (start 104.882298 89.662) (end 104.2162 88.995902) (width 0.25) (layer B.Cu) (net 6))
 (segment (start 111.0615 88.3412) (end 111.0488 88.3412) (width 0.25) (layer B.Cu) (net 6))
 (segment (start 108.5215 84.3915) (end 108.5215 88.3412) (width 0.25) (layer F.Cu) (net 12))
 (segment (start 105.9246 81.7946) (end 108.5215 84.3915) (width 0.25) (layer F.Cu) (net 12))
 (segment (start 105.9246 78.548601) (end 105.9246 81.7946) (width 0.25) (layer F.Cu) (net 12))
 (segment (start 114.313599 74.738601) (end 112.205399 74.738601) (width 0.4) (layer B.Cu) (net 5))
 (via (at 121.158 74.7395) (size 0.8) (drill 0.4) (layers F.Cu B.Cu) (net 5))
 (segment (start 119.3946 74.738601) (end 119.344699 74.6887) (width 0.4) (layer F.Cu) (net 5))
 (segment (start 113.5446 67.118601) (end 113.5446 72.739) (width 0.4) (layer F.Cu) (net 5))
 (segment (start 113.5446 69.9201) (end 113.5446 67.118601) (width 0.4) (layer F.Cu) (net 5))
 (segment (start 118.3132 74.6887) (end 113.5446 69.9201) (width 0.4) (layer F.Cu) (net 5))
 (segment (start 105.9815 80.9625) (end 112.205399 74.738601) (width 0.4) (layer B.Cu) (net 5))
 (segment (start 105.9815 88.3412) (end 105.9815 80.9625) (width 0.4) (layer B.Cu) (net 5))
 (segment (start 121.157101 74.738601) (end 121.158 74.7395) (width 0.4) (layer F.Cu) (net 5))
 (segment (start 119.3946 74.738601) (end 121.157101 74.738601) (width 0.4) (layer F.Cu) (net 5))
 (segment (start 112.2045 74.7395) (end 105.9815 80.9625) (width 0.4) (layer B.Cu) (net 5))
 (segment (start 121.158 74.7395) (end 112.2045 74.7395) (width 0.4) (layer B.Cu) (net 5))
 (segment (start 111.0046 67.945785) (end 111.0046 67.118601) (width 0.4) (layer F.Cu) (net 5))
 (segment (start 119.3946 74.738601) (end 117.797416 74.738601) (width 0.4) (layer F.Cu) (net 5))
 (segment (start 111.0046 67.118601) (end 111.0046 65.6524) (width 0.4) (layer F.Cu) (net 5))
 (segment (start 111.0046 65.6524) (end 111.3155 65.3415) (width 0.4) (layer F.Cu) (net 5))
 (segment (start 111.3155 65.3415) (end 112.9665 65.3415) (width 0.4) (layer F.Cu) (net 5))
 (segment (start 113.5446 65.9196) (end 113.5446 67.118601) (width 0.4) (layer F.Cu) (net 5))
 (segment (start 112.9665 65.3415) (end 113.5446 65.9196) (width 0.4) (layer F.Cu) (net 5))
 (via (at 112.4585 69.1515) (size 0.8) (drill 0.4) (layers F.Cu B.Cu) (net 5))
 (segment (start 111.0046 69.1449) (end 110.998 69.1515) (width 0.4) (layer F.Cu) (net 5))
 (segment (start 111.0046 67.118601) (end 111.0046 69.1449) (width 0.4) (layer F.Cu) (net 5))
 (segment (start 111.0112 69.1515) (end 111.0046 69.1449) (width 0.4) (layer F.Cu) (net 5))
 (segment (start 112.268 69.1515) (end 111.0112 69.1515) (width 0.4) (layer F.Cu) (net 5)))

